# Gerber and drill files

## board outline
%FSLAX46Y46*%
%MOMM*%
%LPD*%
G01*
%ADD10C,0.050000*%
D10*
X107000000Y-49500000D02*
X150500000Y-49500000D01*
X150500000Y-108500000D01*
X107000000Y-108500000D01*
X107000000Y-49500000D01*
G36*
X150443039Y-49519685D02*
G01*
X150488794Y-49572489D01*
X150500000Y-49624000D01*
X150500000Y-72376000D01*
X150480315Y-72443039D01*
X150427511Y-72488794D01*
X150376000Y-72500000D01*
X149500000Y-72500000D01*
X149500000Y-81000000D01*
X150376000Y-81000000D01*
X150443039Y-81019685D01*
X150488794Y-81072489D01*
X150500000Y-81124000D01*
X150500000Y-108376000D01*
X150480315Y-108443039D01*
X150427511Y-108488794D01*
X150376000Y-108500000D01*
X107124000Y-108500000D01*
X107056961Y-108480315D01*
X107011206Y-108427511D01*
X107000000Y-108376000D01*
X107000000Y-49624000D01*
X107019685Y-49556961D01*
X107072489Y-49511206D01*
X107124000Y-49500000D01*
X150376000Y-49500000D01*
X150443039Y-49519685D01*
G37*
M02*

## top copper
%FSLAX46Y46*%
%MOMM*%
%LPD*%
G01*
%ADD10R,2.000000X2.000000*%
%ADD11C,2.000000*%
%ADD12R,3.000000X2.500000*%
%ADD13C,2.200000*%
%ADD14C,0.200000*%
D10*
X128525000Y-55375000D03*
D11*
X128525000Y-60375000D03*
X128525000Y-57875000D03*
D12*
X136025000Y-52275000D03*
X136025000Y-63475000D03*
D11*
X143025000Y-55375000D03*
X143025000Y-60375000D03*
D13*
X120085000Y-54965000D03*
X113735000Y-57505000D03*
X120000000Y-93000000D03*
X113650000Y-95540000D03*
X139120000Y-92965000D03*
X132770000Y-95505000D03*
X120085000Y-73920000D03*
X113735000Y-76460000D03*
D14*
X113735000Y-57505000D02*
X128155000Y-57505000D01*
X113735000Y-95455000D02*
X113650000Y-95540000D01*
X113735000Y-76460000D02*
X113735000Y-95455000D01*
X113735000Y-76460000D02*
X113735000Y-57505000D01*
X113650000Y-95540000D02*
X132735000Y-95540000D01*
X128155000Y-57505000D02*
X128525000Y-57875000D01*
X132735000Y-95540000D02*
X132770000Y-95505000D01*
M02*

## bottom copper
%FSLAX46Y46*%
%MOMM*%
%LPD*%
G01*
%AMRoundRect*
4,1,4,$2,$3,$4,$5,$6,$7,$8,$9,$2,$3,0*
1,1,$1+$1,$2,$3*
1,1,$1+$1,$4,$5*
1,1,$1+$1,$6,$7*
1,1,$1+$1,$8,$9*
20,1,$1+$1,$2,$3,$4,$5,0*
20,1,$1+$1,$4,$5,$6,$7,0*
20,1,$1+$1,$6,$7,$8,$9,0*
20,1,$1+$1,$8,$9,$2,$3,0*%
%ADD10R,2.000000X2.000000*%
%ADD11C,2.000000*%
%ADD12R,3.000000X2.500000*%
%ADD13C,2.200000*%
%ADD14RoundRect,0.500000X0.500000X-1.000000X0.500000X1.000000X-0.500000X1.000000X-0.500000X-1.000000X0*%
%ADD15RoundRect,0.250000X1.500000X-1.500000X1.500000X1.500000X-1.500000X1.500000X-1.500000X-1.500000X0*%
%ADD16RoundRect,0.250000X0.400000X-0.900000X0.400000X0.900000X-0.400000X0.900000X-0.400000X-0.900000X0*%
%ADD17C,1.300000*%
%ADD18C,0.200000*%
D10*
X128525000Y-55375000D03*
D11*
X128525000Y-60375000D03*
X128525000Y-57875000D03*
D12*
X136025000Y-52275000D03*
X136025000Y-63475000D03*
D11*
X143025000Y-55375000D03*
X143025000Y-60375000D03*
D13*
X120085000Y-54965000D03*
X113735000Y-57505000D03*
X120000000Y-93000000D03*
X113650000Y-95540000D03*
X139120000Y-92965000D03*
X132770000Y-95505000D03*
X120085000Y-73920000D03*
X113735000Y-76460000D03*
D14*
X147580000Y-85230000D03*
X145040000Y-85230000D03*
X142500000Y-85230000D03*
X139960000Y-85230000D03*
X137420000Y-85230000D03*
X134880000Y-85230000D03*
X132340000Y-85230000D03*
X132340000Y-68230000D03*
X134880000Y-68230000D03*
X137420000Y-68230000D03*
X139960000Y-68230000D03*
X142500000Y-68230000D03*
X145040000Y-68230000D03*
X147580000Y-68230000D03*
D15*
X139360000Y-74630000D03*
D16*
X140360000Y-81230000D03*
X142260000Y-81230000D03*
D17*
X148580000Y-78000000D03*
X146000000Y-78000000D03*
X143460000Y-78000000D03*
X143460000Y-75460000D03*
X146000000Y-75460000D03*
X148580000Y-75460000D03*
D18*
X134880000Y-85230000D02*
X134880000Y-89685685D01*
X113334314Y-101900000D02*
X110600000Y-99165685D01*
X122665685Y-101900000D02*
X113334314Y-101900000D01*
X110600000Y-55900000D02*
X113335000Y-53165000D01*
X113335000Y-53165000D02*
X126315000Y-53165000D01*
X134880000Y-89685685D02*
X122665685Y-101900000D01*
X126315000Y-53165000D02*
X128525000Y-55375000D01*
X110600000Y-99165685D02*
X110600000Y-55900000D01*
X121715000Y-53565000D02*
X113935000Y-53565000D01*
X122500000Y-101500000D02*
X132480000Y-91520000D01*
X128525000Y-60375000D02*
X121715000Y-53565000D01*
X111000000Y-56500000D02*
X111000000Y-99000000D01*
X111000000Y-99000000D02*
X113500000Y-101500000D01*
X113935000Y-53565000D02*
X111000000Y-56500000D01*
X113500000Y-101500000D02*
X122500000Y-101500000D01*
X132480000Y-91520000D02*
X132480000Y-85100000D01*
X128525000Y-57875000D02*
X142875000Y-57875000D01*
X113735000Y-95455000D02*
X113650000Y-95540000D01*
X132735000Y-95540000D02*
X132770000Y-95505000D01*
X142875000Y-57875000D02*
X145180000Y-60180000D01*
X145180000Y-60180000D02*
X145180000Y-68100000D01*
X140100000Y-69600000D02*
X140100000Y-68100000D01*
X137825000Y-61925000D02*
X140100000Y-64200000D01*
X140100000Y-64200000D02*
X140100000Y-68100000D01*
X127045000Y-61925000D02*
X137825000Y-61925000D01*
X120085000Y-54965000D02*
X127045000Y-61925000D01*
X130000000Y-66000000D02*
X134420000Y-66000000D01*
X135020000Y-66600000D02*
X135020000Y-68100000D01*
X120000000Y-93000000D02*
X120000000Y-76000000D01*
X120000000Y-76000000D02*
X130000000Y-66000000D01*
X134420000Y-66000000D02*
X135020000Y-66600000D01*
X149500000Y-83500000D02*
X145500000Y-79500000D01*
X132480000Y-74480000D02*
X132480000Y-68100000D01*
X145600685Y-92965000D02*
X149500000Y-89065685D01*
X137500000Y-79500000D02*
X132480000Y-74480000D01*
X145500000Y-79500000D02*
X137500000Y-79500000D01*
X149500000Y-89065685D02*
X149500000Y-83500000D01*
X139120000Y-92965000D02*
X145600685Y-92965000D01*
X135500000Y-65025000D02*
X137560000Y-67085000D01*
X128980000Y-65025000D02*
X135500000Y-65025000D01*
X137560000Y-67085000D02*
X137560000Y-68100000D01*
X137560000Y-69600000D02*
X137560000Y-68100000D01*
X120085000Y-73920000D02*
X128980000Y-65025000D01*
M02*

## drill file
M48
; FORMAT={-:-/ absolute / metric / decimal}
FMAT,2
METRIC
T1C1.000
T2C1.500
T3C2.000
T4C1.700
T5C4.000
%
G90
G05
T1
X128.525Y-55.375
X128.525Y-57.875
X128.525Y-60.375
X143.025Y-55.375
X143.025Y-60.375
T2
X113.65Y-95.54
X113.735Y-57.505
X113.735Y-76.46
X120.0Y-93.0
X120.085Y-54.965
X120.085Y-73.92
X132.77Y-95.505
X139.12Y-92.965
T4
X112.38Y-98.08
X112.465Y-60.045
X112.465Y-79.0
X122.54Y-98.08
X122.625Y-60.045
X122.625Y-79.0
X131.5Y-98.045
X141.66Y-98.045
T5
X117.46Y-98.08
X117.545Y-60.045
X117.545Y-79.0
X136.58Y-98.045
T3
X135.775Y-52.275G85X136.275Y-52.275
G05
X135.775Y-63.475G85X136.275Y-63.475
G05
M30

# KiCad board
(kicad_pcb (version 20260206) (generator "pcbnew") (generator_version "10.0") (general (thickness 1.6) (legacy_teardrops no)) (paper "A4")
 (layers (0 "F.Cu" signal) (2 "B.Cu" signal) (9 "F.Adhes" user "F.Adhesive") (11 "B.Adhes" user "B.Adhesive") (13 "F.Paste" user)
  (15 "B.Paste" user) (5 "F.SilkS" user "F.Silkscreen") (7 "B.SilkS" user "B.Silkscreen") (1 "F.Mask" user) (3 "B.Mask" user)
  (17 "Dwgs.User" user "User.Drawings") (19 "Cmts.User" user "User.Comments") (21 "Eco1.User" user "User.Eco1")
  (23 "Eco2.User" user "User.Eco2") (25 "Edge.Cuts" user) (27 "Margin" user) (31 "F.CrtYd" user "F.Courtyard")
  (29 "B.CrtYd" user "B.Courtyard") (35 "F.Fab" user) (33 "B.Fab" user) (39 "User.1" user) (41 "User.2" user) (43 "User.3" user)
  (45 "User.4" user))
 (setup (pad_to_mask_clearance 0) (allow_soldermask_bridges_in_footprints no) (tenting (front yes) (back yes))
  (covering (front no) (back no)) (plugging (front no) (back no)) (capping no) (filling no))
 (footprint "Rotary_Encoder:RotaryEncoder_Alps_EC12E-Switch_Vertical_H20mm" (layer "F.Cu") (at 128.525 55.375)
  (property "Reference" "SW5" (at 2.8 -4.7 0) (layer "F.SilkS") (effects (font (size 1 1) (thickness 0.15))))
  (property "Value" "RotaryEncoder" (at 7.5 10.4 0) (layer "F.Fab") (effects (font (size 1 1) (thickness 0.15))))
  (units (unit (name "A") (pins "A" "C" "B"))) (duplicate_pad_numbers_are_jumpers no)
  (pad "A" thru_hole rect (at 0 0) (size 2 2) (drill 1) (layers "*.Cu" "*.Mask") (remove_unused_layers no) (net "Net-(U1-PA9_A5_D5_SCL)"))
  (pad "B" thru_hole circle (at 0 5) (size 2 2) (drill 1) (layers "*.Cu" "*.Mask") (remove_unused_layers no) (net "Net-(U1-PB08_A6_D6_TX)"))
  (pad "C" thru_hole circle (at 0 2.5) (size 2 2) (drill 1) (layers "*.Cu" "*.Mask") (remove_unused_layers no) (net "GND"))
  (pad "MP" thru_hole rect (at 7.5 -3.1) (size 3 2.5) (drill oval 2.5 2) (layers "*.Cu" "*.Mask") (remove_unused_layers no))
  (pad "MP" thru_hole rect (at 7.5 8.1) (size 3 2.5) (drill oval 2.5 2) (layers "*.Cu" "*.Mask") (remove_unused_layers no))
  (pad "S1" thru_hole circle (at 14.5 0) (size 2 2) (drill 1) (layers "*.Cu" "*.Mask") (remove_unused_layers no))
  (pad "S2" thru_hole circle (at 14.5 5) (size 2 2) (drill 1) (layers "*.Cu" "*.Mask") (remove_unused_layers no)))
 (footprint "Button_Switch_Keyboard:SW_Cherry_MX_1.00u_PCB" (layer "F.Cu") (at 120.085 54.965)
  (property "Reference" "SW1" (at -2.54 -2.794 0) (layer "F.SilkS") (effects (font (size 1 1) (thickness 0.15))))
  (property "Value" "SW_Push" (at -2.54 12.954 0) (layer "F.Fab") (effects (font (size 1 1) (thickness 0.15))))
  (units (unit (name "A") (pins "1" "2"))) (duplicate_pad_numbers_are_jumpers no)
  (pad "" np_thru_hole circle (at -7.62 5.08) (size 1.7 1.7) (drill 1.7) (layers "*.Cu" "*.Mask"))
  (pad "" np_thru_hole circle (at -2.54 5.08) (size 4 4) (drill 4) (layers "*.Cu" "*.Mask"))
  (pad "" np_thru_hole circle (at 2.54 5.08) (size 1.7 1.7) (drill 1.7) (layers "*.Cu" "*.Mask"))
  (pad "1" thru_hole circle (at 0 0) (size 2.2 2.2) (drill 1.5) (layers "*.Cu" "*.Mask") (remove_unused_layers no)
   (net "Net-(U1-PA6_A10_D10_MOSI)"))
  (pad "2" thru_hole circle (at -6.35 2.54) (size 2.2 2.2) (drill 1.5) (layers "*.Cu" "*.Mask") (remove_unused_layers no) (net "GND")))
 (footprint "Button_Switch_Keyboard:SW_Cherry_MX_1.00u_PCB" (layer "F.Cu") (at 120 93)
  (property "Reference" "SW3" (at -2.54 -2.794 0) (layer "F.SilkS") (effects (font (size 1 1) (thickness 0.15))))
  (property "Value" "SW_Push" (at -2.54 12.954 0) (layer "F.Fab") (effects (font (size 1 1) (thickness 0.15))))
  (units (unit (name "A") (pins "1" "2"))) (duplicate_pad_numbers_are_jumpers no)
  (pad "" np_thru_hole circle (at -7.62 5.08) (size 1.7 1.7) (drill 1.7) (layers "*.Cu" "*.Mask"))
  (pad "" np_thru_hole circle (at -2.54 5.08) (size 4 4) (drill 4) (layers "*.Cu" "*.Mask"))
  (pad "" np_thru_hole circle (at 2.54 5.08) (size 1.7 1.7) (drill 1.7) (layers "*.Cu" "*.Mask"))
  (pad "1" thru_hole circle (at 0 0) (size 2.2 2.2) (drill 1.5) (layers "*.Cu" "*.Mask") (remove_unused_layers no)
   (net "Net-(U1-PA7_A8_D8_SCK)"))
  (pad "2" thru_hole circle (at -6.35 2.54) (size 2.2 2.2) (drill 1.5) (layers "*.Cu" "*.Mask") (remove_unused_layers no) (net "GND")))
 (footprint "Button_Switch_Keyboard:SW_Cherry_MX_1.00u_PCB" (layer "F.Cu") (at 139.12 92.965)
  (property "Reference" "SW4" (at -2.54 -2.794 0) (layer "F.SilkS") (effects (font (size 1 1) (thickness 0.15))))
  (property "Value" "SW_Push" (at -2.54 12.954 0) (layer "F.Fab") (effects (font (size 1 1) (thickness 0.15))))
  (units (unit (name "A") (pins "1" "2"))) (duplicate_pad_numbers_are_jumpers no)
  (pad "" np_thru_hole circle (at -7.62 5.08) (size 1.7 1.7) (drill 1.7) (layers "*.Cu" "*.Mask"))
  (pad "" np_thru_hole circle (at -2.54 5.08) (size 4 4) (drill 4) (layers "*.Cu" "*.Mask"))
  (pad "" np_thru_hole circle (at 2.54 5.08) (size 1.7 1.7) (drill 1.7) (layers "*.Cu" "*.Mask"))
  (pad "1" thru_hole circle (at 0 0) (size 2.2 2.2) (drill 1.5) (layers "*.Cu" "*.Mask") (remove_unused_layers no)
   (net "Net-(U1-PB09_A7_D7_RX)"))
  (pad "2" thru_hole circle (at -6.35 2.54) (size 2.2 2.2) (drill 1.5) (layers "*.Cu" "*.Mask") (remove_unused_layers no) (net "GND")))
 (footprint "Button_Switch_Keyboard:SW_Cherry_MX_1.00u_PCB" (layer "F.Cu") (at 120.085 73.92)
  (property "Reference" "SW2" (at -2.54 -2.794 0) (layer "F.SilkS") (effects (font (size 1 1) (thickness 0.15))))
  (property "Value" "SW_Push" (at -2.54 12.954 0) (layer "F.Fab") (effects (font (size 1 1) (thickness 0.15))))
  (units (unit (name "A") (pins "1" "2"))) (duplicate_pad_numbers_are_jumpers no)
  (pad "" np_thru_hole circle (at -7.62 5.08) (size 1.7 1.7) (drill 1.7) (layers "*.Cu" "*.Mask"))
  (pad "" np_thru_hole circle (at -2.54 5.08) (size 4 4) (drill 4) (layers "*.Cu" "*.Mask"))
  (pad "" np_thru_hole circle (at 2.54 5.08) (size 1.7 1.7) (drill 1.7) (layers "*.Cu" "*.Mask"))
  (pad "1" thru_hole circle (at 0 0) (size 2.2 2.2) (drill 1.5) (layers "*.Cu" "*.Mask") (remove_unused_layers no)
   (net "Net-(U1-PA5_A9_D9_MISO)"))
  (pad "2" thru_hole circle (at -6.35 2.54) (size 2.2 2.2) (drill 1.5) (layers "*.Cu" "*.Mask") (remove_unused_layers no) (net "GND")))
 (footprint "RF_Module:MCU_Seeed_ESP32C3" (layer "B.Cu") (at 139.96 76.73 90)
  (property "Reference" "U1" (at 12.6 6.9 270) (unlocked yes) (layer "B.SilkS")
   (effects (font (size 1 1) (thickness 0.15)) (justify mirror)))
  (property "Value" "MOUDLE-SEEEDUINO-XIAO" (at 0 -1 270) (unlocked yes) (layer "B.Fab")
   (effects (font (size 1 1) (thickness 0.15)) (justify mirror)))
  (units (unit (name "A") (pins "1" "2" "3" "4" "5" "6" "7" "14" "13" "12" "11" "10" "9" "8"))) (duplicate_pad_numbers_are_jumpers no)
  (pad "" smd roundrect (at 1.1 -1.6 90) (size 1.5 1.5) (layers "B.Paste") (roundrect_rratio 0.1666666667))
  (pad "" smd roundrect (at 1.1 0.4 90) (size 1.5 1.5) (layers "B.Paste") (roundrect_rratio 0.1666666667))
  (pad "" smd roundrect (at 3.1 -1.6 90) (size 1.5 1.5) (layers "B.Paste") (roundrect_rratio 0.1666666667))
  (pad "" smd roundrect (at 3.1 0.4 90) (size 1.5 1.5) (layers "B.Paste") (roundrect_rratio 0.1666666667))
  (pad "1" smd roundrect (at -8.5 7.62 90) (size 3 2) (layers "B.Cu" "B.Mask" "B.Paste") (roundrect_rratio 0.25)
   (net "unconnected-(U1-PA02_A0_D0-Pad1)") (thermal_bridge_angle 45))
  (pad "2" smd roundrect (at -8.5 5.08 90) (size 3 2) (layers "B.Cu" "B.Mask" "B.Paste") (roundrect_rratio 0.25)
   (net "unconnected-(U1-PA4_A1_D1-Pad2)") (thermal_bridge_angle 45))
  (pad "3" smd roundrect (at -8.5 2.54 90) (size 3 2) (layers "B.Cu" "B.Mask" "B.Paste") (roundrect_rratio 0.25)
   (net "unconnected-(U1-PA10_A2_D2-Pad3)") (thermal_bridge_angle 45))
  (pad "4" smd roundrect (at -8.5 0 90) (size 3 2) (layers "B.Cu" "B.Mask" "B.Paste") (roundrect_rratio 0.25)
   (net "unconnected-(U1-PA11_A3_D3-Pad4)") (thermal_bridge_angle 45))
  (pad "5" smd roundrect (at -8.5 -2.54 90) (size 3 2) (layers "B.Cu" "B.Mask" "B.Paste") (roundrect_rratio 0.25)
   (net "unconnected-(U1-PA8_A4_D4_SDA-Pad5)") (thermal_bridge_angle 45))
  (pad "6" smd roundrect (at -8.5 -5.08 90) (size 3 2) (layers "B.Cu" "B.Mask" "B.Paste") (roundrect_rratio 0.25)
   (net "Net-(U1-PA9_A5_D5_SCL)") (thermal_bridge_angle 45))
  (pad "7" smd roundrect (at -8.5 -7.62 90) (size 3 2) (layers "B.Cu" "B.Mask" "B.Paste") (roundrect_rratio 0.25)
   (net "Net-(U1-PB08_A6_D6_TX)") (thermal_bridge_angle 45))
  (pad "8" smd roundrect (at 8.5 -7.62 90) (size 3 2) (layers "B.Cu" "B.Mask" "B.Paste") (roundrect_rratio 0.25)
   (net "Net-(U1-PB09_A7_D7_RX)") (thermal_bridge_angle 45))
  (pad "9" smd roundrect (at 8.5 -5.08 90) (size 3 2) (layers "B.Cu" "B.Mask" "B.Paste") (roundrect_rratio 0.25)
   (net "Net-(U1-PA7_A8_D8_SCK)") (thermal_bridge_angle 45))
  (pad "10" smd roundrect (at 8.5 -2.54 90) (size 3 2) (layers "B.Cu" "B.Mask" "B.Paste") (roundrect_rratio 0.25)
   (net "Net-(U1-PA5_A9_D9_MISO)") (thermal_bridge_angle 45))
  (pad "11" smd roundrect (at 8.5 0 90) (size 3 2) (layers "B.Cu" "B.Mask" "B.Paste") (roundrect_rratio 0.25)
   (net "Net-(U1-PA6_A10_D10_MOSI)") (thermal_bridge_angle 45))
  (pad "12" smd roundrect (at 8.5 2.54 90) (size 3 2) (layers "B.Cu" "B.Mask" "B.Paste") (roundrect_rratio 0.25)
   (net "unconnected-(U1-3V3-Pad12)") (thermal_bridge_angle 45))
  (pad "13" smd roundrect (at 8.5 5.08 90) (size 3 2) (layers "B.Cu" "B.Mask" "B.Paste") (roundrect_rratio 0.25) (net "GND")
   (thermal_bridge_angle 45))
  (pad "14" smd roundrect (at 8.5 7.62 90) (size 3 2) (layers "B.Cu" "B.Mask" "B.Paste") (roundrect_rratio 0.25)
   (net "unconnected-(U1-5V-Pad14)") (thermal_bridge_angle 45))
  (pad "15" smd roundrect (at 2.1 -0.6 90) (size 3.5 3.5) (layers "B.Cu" "B.Mask") (roundrect_rratio 0.07142857143))
  (pad "16" smd roundrect (at -4.5 0.4 90) (size 2.3 1.3) (layers "B.Cu" "B.Mask" "B.Paste") (roundrect_rratio 0.1923076923))
  (pad "17" smd roundrect (at -4.5 2.3 90) (size 2.3 1.3) (layers "B.Cu" "B.Mask" "B.Paste") (roundrect_rratio 0.1923076923))
  (pad "18" smd circle (at -1.27 8.62 90) (size 1.3 1.3) (layers "B.Cu" "B.Mask" "B.Paste"))
  (pad "19" smd circle (at -1.27 6.04 90) (size 1.3 1.3) (layers "B.Cu" "B.Mask" "B.Paste"))
  (pad "20" smd circle (at -1.27 3.5 90) (size 1.3 1.3) (layers "B.Cu" "B.Mask" "B.Paste"))
  (pad "21" smd circle (at 1.27 3.5 90) (size 1.3 1.3) (layers "B.Cu" "B.Mask" "B.Paste"))
  (pad "22" smd circle (at 1.27 6.04 90) (size 1.3 1.3) (layers "B.Cu" "B.Mask" "B.Paste"))
  (pad "23" smd circle (at 1.27 8.62 90) (size 1.3 1.3) (layers "B.Cu" "B.Mask" "B.Paste")))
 (gr_rect (start 107 49.5) (end 150.5 108.5) (stroke (width 0.05) (type default)) (fill no) (layer "Edge.Cuts"))
 (segment (start 134.88 85.23) (end 134.88 89.685685) (width 0.2) (layer "B.Cu") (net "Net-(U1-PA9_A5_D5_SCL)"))
 (segment (start 113.334314 101.9) (end 110.6 99.165685) (width 0.2) (layer "B.Cu") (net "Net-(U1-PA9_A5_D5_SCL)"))
 (segment (start 122.665685 101.9) (end 113.334314 101.9) (width 0.2) (layer "B.Cu") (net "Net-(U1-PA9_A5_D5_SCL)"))
 (segment (start 110.6 55.9) (end 113.335 53.165) (width 0.2) (layer "B.Cu") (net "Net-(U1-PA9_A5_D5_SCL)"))
 (segment (start 113.335 53.165) (end 126.315 53.165) (width 0.2) (layer "B.Cu") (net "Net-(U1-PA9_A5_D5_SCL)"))
 (segment (start 134.88 89.685685) (end 122.665685 101.9) (width 0.2) (layer "B.Cu") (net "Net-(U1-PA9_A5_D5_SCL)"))
 (segment (start 126.315 53.165) (end 128.525 55.375) (width 0.2) (layer "B.Cu") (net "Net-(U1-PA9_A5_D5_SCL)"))
 (segment (start 110.6 99.165685) (end 110.6 55.9) (width 0.2) (layer "B.Cu") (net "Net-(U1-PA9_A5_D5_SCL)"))
 (segment (start 121.715 53.565) (end 113.935 53.565) (width 0.2) (layer "B.Cu") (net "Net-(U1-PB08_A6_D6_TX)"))
 (segment (start 122.5 101.5) (end 132.48 91.52) (width 0.2) (layer "B.Cu") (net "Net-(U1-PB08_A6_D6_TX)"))
 (segment (start 128.525 60.375) (end 121.715 53.565) (width 0.2) (layer "B.Cu") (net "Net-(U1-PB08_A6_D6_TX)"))
 (segment (start 111 56.5) (end 111 99) (width 0.2) (layer "B.Cu") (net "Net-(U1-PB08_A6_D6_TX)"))
 (segment (start 111 99) (end 113.5 101.5) (width 0.2) (layer "B.Cu") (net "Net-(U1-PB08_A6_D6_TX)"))
 (segment (start 113.935 53.565) (end 111 56.5) (width 0.2) (layer "B.Cu") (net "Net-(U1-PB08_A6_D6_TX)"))
 (segment (start 113.5 101.5) (end 122.5 101.5) (width 0.2) (layer "B.Cu") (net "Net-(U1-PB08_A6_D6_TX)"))
 (segment (start 132.48 91.52) (end 132.48 85.1) (width 0.2) (layer "B.Cu") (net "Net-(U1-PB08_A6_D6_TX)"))
 (segment (start 113.735 57.505) (end 128.155 57.505) (width 0.2) (layer "F.Cu") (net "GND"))
 (segment (start 113.735 95.455) (end 113.65 95.54) (width 0.2) (layer "F.Cu") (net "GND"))
 (segment (start 113.735 76.46) (end 113.735 95.455) (width 0.2) (layer "F.Cu") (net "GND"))
 (segment (start 113.735 76.46) (end 113.735 57.505) (width 0.2) (layer "F.Cu") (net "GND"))
 (segment (start 113.65 95.54) (end 132.735 95.54) (width 0.2) (layer "F.Cu") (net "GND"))
 (segment (start 128.155 57.505) (end 128.525 57.875) (width 0.2) (layer "F.Cu") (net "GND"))
 (segment (start 132.735 95.54) (end 132.77 95.505) (width 0.2) (layer "F.Cu") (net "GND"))
 (segment (start 128.525 57.875) (end 142.875 57.875) (width 0.2) (layer "B.Cu") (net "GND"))
 (segment (start 113.735 95.455) (end 113.65 95.54) (width 0.2) (layer "B.Cu") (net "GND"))
 (segment (start 132.735 95.54) (end 132.77 95.505) (width 0.2) (layer "B.Cu") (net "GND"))
 (segment (start 142.875 57.875) (end 145.18 60.18) (width 0.2) (layer "B.Cu") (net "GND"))
 (segment (start 145.18 60.18) (end 145.18 68.1) (width 0.2) (layer "B.Cu") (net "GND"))
 (segment (start 140.1 69.6) (end 140.1 68.1) (width 0.2) (layer "B.Cu") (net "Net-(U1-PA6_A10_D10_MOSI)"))
 (segment (start 137.825 61.925) (end 140.1 64.2) (width 0.2) (layer "B.Cu") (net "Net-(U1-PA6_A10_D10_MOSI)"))
 (segment (start 140.1 64.2) (end 140.1 68.1) (width 0.2) (layer "B.Cu") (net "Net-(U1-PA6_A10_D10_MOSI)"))
 (segment (start 127.045 61.925) (end 137.825 61.925) (width 0.2) (layer "B.Cu") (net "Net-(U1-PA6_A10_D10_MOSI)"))
 (segment (start 120.085 54.965) (end 127.045 61.925) (width 0.2) (layer "B.Cu") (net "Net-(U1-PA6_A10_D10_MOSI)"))
 (segment (start 130 66) (end 134.42 66) (width 0.2) (layer "B.Cu") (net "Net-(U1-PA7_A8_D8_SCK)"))
 (segment (start 135.02 66.6) (end 135.02 68.1) (width 0.2) (layer "B.Cu") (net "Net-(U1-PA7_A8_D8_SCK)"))
 (segment (start 120 93) (end 120 76) (width 0.2) (layer "B.Cu") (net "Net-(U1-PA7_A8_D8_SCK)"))
 (segment (start 120 76) (end 130 66) (width 0.2) (layer "B.Cu") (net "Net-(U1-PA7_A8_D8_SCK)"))
 (segment (start 134.42 66) (end 135.02 66.6) (width 0.2) (layer "B.Cu") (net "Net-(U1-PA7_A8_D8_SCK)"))
 (segment (start 149.5 83.5) (end 145.5 79.5) (width 0.2) (layer "B.Cu") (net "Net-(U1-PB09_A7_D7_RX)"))
 (segment (start 132.48 74.48) (end 132.48 68.1) (width 0.2) (layer "B.Cu") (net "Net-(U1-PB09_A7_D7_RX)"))
 (segment (start 145.600685 92.965) (end 149.5 89.065685) (width 0.2) (layer "B.Cu") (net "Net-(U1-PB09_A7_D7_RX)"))
 (segment (start 137.5 79.5) (end 132.48 74.48) (width 0.2) (layer "B.Cu") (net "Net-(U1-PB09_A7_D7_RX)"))
 (segment (start 145.5 79.5) (end 137.5 79.5) (width 0.2) (layer "B.Cu") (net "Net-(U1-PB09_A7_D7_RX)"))
 (segment (start 149.5 89.065685) (end 149.5 83.5) (width 0.2) (layer "B.Cu") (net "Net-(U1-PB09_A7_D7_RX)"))
 (segment (start 139.12 92.965) (end 145.600685 92.965) (width 0.2) (layer "B.Cu") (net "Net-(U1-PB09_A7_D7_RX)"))
 (segment (start 135.5 65.025) (end 137.56 67.085) (width 0.2) (layer "B.Cu") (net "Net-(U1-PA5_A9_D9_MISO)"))
 (segment (start 128.98 65.025) (end 135.5 65.025) (width 0.2) (layer "B.Cu") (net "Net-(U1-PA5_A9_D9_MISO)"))
 (segment (start 137.56 67.085) (end 137.56 68.1) (width 0.2) (layer "B.Cu") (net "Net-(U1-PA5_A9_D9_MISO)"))
 (segment (start 137.56 69.6) (end 137.56 68.1) (width 0.2) (layer "B.Cu") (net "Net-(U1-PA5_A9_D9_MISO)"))
 (segment (start 120.085 73.92) (end 128.98 65.025) (width 0.2) (layer "B.Cu") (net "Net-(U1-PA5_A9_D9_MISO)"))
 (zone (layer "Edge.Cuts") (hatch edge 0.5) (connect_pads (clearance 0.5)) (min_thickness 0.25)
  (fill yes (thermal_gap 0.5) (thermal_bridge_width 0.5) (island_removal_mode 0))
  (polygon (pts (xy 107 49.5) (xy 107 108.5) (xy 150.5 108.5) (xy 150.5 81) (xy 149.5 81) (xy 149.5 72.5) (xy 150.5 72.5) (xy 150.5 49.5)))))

